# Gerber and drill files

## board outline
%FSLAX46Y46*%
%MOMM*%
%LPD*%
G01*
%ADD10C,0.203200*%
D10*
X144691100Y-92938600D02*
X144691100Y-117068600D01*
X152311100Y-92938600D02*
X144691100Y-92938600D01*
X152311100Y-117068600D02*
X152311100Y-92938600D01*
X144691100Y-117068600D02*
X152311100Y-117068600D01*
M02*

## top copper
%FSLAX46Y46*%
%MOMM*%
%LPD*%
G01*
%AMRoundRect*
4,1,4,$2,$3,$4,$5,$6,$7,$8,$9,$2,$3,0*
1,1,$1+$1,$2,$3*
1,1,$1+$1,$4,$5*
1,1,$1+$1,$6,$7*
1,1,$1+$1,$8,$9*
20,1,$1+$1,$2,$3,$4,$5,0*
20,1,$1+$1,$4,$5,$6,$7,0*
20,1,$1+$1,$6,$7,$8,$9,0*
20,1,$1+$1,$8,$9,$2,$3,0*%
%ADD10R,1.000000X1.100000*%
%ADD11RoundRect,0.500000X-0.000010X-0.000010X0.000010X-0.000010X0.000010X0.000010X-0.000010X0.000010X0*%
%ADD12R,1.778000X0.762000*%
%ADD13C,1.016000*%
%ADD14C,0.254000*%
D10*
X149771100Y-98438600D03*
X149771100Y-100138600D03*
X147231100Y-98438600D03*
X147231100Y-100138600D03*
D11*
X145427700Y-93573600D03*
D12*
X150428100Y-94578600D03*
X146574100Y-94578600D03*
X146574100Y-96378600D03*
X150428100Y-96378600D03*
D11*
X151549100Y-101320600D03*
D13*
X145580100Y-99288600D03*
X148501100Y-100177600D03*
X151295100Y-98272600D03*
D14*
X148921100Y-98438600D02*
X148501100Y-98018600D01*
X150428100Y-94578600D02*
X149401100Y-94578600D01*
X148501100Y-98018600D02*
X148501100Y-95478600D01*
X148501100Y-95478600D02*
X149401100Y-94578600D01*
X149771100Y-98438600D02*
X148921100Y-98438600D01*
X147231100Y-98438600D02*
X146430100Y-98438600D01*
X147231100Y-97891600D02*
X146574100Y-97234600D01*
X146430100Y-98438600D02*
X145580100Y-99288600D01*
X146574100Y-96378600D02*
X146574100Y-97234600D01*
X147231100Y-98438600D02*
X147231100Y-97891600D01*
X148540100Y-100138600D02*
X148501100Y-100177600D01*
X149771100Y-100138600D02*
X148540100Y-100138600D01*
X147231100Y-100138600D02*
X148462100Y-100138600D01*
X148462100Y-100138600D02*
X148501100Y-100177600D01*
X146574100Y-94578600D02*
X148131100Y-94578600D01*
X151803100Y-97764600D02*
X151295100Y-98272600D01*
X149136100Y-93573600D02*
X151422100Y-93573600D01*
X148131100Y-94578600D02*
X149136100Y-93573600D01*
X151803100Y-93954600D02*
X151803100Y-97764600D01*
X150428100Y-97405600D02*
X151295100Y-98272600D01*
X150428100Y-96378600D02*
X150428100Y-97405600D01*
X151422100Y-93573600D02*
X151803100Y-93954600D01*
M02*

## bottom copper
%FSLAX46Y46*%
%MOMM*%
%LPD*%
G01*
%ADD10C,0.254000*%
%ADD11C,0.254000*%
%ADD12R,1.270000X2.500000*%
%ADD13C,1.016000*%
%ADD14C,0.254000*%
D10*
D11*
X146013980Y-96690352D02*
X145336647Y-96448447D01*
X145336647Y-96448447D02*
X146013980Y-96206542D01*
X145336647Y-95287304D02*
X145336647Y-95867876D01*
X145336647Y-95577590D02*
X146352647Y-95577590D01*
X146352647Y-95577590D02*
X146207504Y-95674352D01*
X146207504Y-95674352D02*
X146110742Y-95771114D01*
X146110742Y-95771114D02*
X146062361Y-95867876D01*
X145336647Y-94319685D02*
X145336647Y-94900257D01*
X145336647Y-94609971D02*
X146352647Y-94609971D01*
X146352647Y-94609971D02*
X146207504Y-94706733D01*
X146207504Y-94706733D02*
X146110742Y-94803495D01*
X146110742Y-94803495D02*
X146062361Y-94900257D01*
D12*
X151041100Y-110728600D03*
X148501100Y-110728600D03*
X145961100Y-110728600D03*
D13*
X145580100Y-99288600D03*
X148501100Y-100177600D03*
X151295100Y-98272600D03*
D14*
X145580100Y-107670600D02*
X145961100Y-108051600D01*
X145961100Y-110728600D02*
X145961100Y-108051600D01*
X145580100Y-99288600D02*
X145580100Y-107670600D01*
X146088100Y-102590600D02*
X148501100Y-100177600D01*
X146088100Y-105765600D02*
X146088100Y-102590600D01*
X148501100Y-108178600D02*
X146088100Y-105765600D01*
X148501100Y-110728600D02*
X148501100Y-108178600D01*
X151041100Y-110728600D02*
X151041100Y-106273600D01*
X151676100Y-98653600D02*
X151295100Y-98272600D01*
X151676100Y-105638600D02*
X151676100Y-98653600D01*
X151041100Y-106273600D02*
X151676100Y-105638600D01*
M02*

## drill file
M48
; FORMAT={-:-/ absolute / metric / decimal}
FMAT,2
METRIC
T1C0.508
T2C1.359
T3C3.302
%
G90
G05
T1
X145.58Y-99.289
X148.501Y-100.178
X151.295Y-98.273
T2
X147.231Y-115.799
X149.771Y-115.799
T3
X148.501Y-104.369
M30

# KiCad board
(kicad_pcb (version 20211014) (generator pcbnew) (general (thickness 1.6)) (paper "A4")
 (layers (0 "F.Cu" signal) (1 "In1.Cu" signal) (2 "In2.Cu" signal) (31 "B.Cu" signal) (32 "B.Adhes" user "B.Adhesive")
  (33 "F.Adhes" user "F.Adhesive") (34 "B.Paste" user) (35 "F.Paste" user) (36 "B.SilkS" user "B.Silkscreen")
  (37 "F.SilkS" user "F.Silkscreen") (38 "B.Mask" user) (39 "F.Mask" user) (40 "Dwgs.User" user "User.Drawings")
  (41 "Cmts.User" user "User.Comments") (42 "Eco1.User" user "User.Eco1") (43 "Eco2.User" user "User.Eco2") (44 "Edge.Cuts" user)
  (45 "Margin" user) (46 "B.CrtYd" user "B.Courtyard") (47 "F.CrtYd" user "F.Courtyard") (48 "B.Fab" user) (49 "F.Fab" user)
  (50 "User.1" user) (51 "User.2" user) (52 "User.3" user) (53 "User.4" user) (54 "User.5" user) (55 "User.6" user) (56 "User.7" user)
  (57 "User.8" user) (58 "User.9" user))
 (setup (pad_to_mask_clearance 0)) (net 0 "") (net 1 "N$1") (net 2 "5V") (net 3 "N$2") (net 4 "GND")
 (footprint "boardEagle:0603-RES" (layer "F.Cu") (at 149.7711 99.2886 -90)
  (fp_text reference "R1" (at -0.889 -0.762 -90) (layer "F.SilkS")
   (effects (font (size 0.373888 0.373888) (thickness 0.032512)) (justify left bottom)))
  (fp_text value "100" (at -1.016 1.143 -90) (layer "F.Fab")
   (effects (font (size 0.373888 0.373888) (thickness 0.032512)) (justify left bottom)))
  (pad "1" smd rect (at -0.85 0 270) (size 1.1 1) (layers "F.Cu" "F.Paste" "F.Mask") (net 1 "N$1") (solder_mask_margin 0.1016))
  (pad "2" smd rect (at 0.85 0 270) (size 1.1 1) (layers "F.Cu" "F.Paste" "F.Mask") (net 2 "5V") (solder_mask_margin 0.1016)))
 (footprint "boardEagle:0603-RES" (layer "F.Cu") (at 147.2311 99.2886 -90)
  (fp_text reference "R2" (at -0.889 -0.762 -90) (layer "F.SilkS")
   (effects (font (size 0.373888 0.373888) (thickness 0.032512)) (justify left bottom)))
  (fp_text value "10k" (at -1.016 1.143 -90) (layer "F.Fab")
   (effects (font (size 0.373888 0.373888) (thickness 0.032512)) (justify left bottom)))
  (pad "1" smd rect (at -0.85 0 270) (size 1.1 1) (layers "F.Cu" "F.Paste" "F.Mask") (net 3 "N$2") (solder_mask_margin 0.1016))
  (pad "2" smd rect (at 0.85 0 270) (size 1.1 1) (layers "F.Cu" "F.Paste" "F.Mask") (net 2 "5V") (solder_mask_margin 0.1016)))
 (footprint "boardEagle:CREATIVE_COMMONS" (layer "F.Cu") (at 119.2911 131.0386)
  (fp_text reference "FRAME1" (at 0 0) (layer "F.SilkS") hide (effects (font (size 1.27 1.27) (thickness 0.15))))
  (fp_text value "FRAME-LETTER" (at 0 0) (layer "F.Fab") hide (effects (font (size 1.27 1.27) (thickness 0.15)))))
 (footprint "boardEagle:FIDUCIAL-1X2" (layer "F.Cu") (at 145.4277 93.5736)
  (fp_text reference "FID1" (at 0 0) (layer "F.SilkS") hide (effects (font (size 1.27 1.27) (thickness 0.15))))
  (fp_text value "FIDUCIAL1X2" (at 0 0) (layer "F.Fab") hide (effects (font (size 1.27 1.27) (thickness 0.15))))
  (pad "1" smd roundrect (at 0 0) (size 1 1) (layers "F.Cu" "F.Mask") (roundrect_rratio 0.5) (solder_mask_margin 0.1016)))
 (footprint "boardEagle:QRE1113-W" (layer "F.Cu") (at 148.5011 95.4786 180)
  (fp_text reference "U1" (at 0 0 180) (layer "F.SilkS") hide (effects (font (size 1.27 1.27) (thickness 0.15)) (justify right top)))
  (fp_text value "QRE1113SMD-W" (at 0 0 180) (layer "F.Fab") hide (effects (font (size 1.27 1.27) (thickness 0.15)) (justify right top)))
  (pad "1" smd rect (at -1.927 0.9 180) (size 1.778 0.762) (layers "F.Cu" "F.Paste" "F.Mask") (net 1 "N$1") (solder_mask_margin 0.1016))
  (pad "2" smd rect (at 1.927 0.9 180) (size 1.778 0.762) (layers "F.Cu" "F.Paste" "F.Mask") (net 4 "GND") (solder_mask_margin 0.1016))
  (pad "3" smd rect (at 1.927 -0.9 180) (size 1.778 0.762) (layers "F.Cu" "F.Paste" "F.Mask") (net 3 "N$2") (solder_mask_margin 0.1016))
  (pad "4" smd rect (at -1.927 -0.9 180) (size 1.778 0.762) (layers "F.Cu" "F.Paste" "F.Mask") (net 4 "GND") (solder_mask_margin 0.1016)))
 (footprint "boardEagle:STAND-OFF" (layer "F.Cu") (at 148.5011 104.3686)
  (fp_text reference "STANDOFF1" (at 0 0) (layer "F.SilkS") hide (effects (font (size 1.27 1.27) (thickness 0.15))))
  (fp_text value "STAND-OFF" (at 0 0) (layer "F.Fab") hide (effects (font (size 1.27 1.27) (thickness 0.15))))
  (pad "" np_thru_hole circle (at 0 0) (size 3.302 3.302) (drill 3.302) (layers *.Cu *.Mask)))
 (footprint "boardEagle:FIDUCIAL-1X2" (layer "F.Cu") (at 151.5491 101.3206)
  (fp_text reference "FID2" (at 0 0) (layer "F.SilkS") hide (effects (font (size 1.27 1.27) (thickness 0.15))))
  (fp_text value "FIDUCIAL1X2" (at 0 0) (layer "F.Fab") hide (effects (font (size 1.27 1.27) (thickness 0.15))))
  (pad "1" smd roundrect (at 0 0) (size 1 1) (layers "F.Cu" "F.Mask") (roundrect_rratio 0.5) (solder_mask_margin 0.1016)))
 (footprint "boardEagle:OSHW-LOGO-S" (layer "B.Cu") (at 148.5011 95.4786 180)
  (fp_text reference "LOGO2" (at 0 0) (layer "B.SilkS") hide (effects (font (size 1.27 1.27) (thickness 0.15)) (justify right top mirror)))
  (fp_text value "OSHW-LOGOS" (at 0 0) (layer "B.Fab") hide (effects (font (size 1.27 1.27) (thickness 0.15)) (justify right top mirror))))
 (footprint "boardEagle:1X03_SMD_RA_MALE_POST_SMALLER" (layer "B.Cu") (at 148.5011 115.7986 180)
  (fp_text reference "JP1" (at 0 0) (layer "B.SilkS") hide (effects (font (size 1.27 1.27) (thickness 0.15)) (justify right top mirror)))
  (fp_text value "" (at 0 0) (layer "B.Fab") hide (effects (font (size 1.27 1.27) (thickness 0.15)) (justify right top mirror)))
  (pad "" np_thru_hole circle (at 1.27 0 180) (size 1.3589 1.3589) (drill 1.3589) (layers *.Cu *.Mask))
  (pad "" np_thru_hole circle (at -1.27 0 180) (size 1.3589 1.3589) (drill 1.3589) (layers *.Cu *.Mask))
  (pad "1" smd rect (at -2.54 5.07 90) (size 2.5 1.27) (layers "B.Cu" "B.Paste" "B.Mask") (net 4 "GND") (solder_mask_margin 0.1016))
  (pad "2" smd rect (at 0 5.07 90) (size 2.5 1.27) (layers "B.Cu" "B.Paste" "B.Mask") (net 2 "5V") (solder_mask_margin 0.1016))
  (pad "3" smd rect (at 2.54 5.07 90) (size 2.5 1.27) (layers "B.Cu" "B.Paste" "B.Mask") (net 3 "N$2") (solder_mask_margin 0.1016)))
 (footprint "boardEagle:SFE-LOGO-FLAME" (layer "B.Cu") (at 149.5171 99.7966 180)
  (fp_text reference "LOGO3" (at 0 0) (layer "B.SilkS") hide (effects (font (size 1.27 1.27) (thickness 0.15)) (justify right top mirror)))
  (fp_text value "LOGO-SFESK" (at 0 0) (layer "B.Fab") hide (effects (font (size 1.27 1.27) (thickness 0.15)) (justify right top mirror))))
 (gr_line (start 144.6911 92.9386) (end 144.6911 117.0686) (layer "Edge.Cuts") (width 0.2032))
 (gr_line (start 152.3111 92.9386) (end 144.6911 92.9386) (layer "Edge.Cuts") (width 0.2032))
 (gr_line (start 152.3111 117.0686) (end 152.3111 92.9386) (layer "Edge.Cuts") (width 0.2032))
 (gr_line (start 144.6911 117.0686) (end 152.3111 117.0686) (layer "Edge.Cuts") (width 0.2032))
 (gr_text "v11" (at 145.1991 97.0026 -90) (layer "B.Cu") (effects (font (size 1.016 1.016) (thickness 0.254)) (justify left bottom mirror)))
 (segment (start 148.9211 98.4386) (end 148.5011 98.0186) (width 0.254) (layer "F.Cu") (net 1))
 (segment (start 150.4281 94.5786) (end 149.4011 94.5786) (width 0.254) (layer "F.Cu") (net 1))
 (segment (start 148.5011 98.0186) (end 148.5011 95.4786) (width 0.254) (layer "F.Cu") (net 1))
 (segment (start 148.5011 95.4786) (end 149.4011 94.5786) (width 0.254) (layer "F.Cu") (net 1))
 (segment (start 149.7711 98.4386) (end 148.9211 98.4386) (width 0.254) (layer "F.Cu") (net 1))
 (segment (start 147.2311 98.4386) (end 146.4301 98.4386) (width 0.254) (layer "F.Cu") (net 3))
 (segment (start 147.2311 97.8916) (end 146.5741 97.2346) (width 0.254) (layer "F.Cu") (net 3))
 (segment (start 146.4301 98.4386) (end 145.5801 99.2886) (width 0.254) (layer "F.Cu") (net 3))
 (segment (start 146.5741 96.3786) (end 146.5741 97.2346) (width 0.254) (layer "F.Cu") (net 3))
 (segment (start 147.2311 98.4386) (end 147.2311 97.8916) (width 0.254) (layer "F.Cu") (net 3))
 (via (at 145.5801 99.2886) (size 1.016) (drill 0.508) (layers "F.Cu" "B.Cu") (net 3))
 (segment (start 145.5801 107.6706) (end 145.9611 108.0516) (width 0.254) (layer "B.Cu") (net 3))
 (segment (start 145.9611 110.7286) (end 145.9611 108.0516) (width 0.254) (layer "B.Cu") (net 3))
 (segment (start 145.5801 99.2886) (end 145.5801 107.6706) (width 0.254) (layer "B.Cu") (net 3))
 (segment (start 148.5401 100.1386) (end 148.5011 100.1776) (width 0.254) (layer "F.Cu") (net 2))
 (segment (start 149.7711 100.1386) (end 148.5401 100.1386) (width 0.254) (layer "F.Cu") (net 2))
 (segment (start 147.2311 100.1386) (end 148.4621 100.1386) (width 0.254) (layer "F.Cu") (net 2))
 (segment (start 148.4621 100.1386) (end 148.5011 100.1776) (width 0.254) (layer "F.Cu") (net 2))
 (via (at 148.5011 100.1776) (size 1.016) (drill 0.508) (layers "F.Cu" "B.Cu") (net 2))
 (segment (start 146.0881 102.5906) (end 148.5011 100.1776) (width 0.254) (layer "B.Cu") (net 2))
 (segment (start 146.0881 105.7656) (end 146.0881 102.5906) (width 0.254) (layer "B.Cu") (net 2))
 (segment (start 148.5011 108.1786) (end 146.0881 105.7656) (width 0.254) (layer "B.Cu") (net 2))
 (segment (start 148.5011 110.7286) (end 148.5011 108.1786) (width 0.254) (layer "B.Cu") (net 2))
 (segment (start 146.5741 94.5786) (end 148.1311 94.5786) (width 0.254) (layer "F.Cu") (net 4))
 (segment (start 151.8031 97.7646) (end 151.2951 98.2726) (width 0.254) (layer "F.Cu") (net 4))
 (segment (start 149.1361 93.5736) (end 151.4221 93.5736) (width 0.254) (layer "F.Cu") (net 4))
 (segment (start 148.1311 94.5786) (end 149.1361 93.5736) (width 0.254) (layer "F.Cu") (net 4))
 (segment (start 151.8031 93.9546) (end 151.8031 97.7646) (width 0.254) (layer "F.Cu") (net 4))
 (segment (start 150.4281 97.4056) (end 151.2951 98.2726) (width 0.254) (layer "F.Cu") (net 4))
 (segment (start 150.4281 96.3786) (end 150.4281 97.4056) (width 0.254) (layer "F.Cu") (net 4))
 (segment (start 151.4221 93.5736) (end 151.8031 93.9546) (width 0.254) (layer "F.Cu") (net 4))
 (via (at 151.2951 98.2726) (size 1.016) (drill 0.508) (layers "F.Cu" "B.Cu") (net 4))
 (segment (start 151.0411 110.7286) (end 151.0411 106.2736) (width 0.254) (layer "B.Cu") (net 4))
 (segment (start 151.6761 98.6536) (end 151.2951 98.2726) (width 0.254) (layer "B.Cu") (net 4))
 (segment (start 151.6761 105.6386) (end 151.6761 98.6536) (width 0.254) (layer "B.Cu") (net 4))
 (segment (start 151.0411 106.2736) (end 151.6761 105.6386) (width 0.254) (layer "B.Cu") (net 4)))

